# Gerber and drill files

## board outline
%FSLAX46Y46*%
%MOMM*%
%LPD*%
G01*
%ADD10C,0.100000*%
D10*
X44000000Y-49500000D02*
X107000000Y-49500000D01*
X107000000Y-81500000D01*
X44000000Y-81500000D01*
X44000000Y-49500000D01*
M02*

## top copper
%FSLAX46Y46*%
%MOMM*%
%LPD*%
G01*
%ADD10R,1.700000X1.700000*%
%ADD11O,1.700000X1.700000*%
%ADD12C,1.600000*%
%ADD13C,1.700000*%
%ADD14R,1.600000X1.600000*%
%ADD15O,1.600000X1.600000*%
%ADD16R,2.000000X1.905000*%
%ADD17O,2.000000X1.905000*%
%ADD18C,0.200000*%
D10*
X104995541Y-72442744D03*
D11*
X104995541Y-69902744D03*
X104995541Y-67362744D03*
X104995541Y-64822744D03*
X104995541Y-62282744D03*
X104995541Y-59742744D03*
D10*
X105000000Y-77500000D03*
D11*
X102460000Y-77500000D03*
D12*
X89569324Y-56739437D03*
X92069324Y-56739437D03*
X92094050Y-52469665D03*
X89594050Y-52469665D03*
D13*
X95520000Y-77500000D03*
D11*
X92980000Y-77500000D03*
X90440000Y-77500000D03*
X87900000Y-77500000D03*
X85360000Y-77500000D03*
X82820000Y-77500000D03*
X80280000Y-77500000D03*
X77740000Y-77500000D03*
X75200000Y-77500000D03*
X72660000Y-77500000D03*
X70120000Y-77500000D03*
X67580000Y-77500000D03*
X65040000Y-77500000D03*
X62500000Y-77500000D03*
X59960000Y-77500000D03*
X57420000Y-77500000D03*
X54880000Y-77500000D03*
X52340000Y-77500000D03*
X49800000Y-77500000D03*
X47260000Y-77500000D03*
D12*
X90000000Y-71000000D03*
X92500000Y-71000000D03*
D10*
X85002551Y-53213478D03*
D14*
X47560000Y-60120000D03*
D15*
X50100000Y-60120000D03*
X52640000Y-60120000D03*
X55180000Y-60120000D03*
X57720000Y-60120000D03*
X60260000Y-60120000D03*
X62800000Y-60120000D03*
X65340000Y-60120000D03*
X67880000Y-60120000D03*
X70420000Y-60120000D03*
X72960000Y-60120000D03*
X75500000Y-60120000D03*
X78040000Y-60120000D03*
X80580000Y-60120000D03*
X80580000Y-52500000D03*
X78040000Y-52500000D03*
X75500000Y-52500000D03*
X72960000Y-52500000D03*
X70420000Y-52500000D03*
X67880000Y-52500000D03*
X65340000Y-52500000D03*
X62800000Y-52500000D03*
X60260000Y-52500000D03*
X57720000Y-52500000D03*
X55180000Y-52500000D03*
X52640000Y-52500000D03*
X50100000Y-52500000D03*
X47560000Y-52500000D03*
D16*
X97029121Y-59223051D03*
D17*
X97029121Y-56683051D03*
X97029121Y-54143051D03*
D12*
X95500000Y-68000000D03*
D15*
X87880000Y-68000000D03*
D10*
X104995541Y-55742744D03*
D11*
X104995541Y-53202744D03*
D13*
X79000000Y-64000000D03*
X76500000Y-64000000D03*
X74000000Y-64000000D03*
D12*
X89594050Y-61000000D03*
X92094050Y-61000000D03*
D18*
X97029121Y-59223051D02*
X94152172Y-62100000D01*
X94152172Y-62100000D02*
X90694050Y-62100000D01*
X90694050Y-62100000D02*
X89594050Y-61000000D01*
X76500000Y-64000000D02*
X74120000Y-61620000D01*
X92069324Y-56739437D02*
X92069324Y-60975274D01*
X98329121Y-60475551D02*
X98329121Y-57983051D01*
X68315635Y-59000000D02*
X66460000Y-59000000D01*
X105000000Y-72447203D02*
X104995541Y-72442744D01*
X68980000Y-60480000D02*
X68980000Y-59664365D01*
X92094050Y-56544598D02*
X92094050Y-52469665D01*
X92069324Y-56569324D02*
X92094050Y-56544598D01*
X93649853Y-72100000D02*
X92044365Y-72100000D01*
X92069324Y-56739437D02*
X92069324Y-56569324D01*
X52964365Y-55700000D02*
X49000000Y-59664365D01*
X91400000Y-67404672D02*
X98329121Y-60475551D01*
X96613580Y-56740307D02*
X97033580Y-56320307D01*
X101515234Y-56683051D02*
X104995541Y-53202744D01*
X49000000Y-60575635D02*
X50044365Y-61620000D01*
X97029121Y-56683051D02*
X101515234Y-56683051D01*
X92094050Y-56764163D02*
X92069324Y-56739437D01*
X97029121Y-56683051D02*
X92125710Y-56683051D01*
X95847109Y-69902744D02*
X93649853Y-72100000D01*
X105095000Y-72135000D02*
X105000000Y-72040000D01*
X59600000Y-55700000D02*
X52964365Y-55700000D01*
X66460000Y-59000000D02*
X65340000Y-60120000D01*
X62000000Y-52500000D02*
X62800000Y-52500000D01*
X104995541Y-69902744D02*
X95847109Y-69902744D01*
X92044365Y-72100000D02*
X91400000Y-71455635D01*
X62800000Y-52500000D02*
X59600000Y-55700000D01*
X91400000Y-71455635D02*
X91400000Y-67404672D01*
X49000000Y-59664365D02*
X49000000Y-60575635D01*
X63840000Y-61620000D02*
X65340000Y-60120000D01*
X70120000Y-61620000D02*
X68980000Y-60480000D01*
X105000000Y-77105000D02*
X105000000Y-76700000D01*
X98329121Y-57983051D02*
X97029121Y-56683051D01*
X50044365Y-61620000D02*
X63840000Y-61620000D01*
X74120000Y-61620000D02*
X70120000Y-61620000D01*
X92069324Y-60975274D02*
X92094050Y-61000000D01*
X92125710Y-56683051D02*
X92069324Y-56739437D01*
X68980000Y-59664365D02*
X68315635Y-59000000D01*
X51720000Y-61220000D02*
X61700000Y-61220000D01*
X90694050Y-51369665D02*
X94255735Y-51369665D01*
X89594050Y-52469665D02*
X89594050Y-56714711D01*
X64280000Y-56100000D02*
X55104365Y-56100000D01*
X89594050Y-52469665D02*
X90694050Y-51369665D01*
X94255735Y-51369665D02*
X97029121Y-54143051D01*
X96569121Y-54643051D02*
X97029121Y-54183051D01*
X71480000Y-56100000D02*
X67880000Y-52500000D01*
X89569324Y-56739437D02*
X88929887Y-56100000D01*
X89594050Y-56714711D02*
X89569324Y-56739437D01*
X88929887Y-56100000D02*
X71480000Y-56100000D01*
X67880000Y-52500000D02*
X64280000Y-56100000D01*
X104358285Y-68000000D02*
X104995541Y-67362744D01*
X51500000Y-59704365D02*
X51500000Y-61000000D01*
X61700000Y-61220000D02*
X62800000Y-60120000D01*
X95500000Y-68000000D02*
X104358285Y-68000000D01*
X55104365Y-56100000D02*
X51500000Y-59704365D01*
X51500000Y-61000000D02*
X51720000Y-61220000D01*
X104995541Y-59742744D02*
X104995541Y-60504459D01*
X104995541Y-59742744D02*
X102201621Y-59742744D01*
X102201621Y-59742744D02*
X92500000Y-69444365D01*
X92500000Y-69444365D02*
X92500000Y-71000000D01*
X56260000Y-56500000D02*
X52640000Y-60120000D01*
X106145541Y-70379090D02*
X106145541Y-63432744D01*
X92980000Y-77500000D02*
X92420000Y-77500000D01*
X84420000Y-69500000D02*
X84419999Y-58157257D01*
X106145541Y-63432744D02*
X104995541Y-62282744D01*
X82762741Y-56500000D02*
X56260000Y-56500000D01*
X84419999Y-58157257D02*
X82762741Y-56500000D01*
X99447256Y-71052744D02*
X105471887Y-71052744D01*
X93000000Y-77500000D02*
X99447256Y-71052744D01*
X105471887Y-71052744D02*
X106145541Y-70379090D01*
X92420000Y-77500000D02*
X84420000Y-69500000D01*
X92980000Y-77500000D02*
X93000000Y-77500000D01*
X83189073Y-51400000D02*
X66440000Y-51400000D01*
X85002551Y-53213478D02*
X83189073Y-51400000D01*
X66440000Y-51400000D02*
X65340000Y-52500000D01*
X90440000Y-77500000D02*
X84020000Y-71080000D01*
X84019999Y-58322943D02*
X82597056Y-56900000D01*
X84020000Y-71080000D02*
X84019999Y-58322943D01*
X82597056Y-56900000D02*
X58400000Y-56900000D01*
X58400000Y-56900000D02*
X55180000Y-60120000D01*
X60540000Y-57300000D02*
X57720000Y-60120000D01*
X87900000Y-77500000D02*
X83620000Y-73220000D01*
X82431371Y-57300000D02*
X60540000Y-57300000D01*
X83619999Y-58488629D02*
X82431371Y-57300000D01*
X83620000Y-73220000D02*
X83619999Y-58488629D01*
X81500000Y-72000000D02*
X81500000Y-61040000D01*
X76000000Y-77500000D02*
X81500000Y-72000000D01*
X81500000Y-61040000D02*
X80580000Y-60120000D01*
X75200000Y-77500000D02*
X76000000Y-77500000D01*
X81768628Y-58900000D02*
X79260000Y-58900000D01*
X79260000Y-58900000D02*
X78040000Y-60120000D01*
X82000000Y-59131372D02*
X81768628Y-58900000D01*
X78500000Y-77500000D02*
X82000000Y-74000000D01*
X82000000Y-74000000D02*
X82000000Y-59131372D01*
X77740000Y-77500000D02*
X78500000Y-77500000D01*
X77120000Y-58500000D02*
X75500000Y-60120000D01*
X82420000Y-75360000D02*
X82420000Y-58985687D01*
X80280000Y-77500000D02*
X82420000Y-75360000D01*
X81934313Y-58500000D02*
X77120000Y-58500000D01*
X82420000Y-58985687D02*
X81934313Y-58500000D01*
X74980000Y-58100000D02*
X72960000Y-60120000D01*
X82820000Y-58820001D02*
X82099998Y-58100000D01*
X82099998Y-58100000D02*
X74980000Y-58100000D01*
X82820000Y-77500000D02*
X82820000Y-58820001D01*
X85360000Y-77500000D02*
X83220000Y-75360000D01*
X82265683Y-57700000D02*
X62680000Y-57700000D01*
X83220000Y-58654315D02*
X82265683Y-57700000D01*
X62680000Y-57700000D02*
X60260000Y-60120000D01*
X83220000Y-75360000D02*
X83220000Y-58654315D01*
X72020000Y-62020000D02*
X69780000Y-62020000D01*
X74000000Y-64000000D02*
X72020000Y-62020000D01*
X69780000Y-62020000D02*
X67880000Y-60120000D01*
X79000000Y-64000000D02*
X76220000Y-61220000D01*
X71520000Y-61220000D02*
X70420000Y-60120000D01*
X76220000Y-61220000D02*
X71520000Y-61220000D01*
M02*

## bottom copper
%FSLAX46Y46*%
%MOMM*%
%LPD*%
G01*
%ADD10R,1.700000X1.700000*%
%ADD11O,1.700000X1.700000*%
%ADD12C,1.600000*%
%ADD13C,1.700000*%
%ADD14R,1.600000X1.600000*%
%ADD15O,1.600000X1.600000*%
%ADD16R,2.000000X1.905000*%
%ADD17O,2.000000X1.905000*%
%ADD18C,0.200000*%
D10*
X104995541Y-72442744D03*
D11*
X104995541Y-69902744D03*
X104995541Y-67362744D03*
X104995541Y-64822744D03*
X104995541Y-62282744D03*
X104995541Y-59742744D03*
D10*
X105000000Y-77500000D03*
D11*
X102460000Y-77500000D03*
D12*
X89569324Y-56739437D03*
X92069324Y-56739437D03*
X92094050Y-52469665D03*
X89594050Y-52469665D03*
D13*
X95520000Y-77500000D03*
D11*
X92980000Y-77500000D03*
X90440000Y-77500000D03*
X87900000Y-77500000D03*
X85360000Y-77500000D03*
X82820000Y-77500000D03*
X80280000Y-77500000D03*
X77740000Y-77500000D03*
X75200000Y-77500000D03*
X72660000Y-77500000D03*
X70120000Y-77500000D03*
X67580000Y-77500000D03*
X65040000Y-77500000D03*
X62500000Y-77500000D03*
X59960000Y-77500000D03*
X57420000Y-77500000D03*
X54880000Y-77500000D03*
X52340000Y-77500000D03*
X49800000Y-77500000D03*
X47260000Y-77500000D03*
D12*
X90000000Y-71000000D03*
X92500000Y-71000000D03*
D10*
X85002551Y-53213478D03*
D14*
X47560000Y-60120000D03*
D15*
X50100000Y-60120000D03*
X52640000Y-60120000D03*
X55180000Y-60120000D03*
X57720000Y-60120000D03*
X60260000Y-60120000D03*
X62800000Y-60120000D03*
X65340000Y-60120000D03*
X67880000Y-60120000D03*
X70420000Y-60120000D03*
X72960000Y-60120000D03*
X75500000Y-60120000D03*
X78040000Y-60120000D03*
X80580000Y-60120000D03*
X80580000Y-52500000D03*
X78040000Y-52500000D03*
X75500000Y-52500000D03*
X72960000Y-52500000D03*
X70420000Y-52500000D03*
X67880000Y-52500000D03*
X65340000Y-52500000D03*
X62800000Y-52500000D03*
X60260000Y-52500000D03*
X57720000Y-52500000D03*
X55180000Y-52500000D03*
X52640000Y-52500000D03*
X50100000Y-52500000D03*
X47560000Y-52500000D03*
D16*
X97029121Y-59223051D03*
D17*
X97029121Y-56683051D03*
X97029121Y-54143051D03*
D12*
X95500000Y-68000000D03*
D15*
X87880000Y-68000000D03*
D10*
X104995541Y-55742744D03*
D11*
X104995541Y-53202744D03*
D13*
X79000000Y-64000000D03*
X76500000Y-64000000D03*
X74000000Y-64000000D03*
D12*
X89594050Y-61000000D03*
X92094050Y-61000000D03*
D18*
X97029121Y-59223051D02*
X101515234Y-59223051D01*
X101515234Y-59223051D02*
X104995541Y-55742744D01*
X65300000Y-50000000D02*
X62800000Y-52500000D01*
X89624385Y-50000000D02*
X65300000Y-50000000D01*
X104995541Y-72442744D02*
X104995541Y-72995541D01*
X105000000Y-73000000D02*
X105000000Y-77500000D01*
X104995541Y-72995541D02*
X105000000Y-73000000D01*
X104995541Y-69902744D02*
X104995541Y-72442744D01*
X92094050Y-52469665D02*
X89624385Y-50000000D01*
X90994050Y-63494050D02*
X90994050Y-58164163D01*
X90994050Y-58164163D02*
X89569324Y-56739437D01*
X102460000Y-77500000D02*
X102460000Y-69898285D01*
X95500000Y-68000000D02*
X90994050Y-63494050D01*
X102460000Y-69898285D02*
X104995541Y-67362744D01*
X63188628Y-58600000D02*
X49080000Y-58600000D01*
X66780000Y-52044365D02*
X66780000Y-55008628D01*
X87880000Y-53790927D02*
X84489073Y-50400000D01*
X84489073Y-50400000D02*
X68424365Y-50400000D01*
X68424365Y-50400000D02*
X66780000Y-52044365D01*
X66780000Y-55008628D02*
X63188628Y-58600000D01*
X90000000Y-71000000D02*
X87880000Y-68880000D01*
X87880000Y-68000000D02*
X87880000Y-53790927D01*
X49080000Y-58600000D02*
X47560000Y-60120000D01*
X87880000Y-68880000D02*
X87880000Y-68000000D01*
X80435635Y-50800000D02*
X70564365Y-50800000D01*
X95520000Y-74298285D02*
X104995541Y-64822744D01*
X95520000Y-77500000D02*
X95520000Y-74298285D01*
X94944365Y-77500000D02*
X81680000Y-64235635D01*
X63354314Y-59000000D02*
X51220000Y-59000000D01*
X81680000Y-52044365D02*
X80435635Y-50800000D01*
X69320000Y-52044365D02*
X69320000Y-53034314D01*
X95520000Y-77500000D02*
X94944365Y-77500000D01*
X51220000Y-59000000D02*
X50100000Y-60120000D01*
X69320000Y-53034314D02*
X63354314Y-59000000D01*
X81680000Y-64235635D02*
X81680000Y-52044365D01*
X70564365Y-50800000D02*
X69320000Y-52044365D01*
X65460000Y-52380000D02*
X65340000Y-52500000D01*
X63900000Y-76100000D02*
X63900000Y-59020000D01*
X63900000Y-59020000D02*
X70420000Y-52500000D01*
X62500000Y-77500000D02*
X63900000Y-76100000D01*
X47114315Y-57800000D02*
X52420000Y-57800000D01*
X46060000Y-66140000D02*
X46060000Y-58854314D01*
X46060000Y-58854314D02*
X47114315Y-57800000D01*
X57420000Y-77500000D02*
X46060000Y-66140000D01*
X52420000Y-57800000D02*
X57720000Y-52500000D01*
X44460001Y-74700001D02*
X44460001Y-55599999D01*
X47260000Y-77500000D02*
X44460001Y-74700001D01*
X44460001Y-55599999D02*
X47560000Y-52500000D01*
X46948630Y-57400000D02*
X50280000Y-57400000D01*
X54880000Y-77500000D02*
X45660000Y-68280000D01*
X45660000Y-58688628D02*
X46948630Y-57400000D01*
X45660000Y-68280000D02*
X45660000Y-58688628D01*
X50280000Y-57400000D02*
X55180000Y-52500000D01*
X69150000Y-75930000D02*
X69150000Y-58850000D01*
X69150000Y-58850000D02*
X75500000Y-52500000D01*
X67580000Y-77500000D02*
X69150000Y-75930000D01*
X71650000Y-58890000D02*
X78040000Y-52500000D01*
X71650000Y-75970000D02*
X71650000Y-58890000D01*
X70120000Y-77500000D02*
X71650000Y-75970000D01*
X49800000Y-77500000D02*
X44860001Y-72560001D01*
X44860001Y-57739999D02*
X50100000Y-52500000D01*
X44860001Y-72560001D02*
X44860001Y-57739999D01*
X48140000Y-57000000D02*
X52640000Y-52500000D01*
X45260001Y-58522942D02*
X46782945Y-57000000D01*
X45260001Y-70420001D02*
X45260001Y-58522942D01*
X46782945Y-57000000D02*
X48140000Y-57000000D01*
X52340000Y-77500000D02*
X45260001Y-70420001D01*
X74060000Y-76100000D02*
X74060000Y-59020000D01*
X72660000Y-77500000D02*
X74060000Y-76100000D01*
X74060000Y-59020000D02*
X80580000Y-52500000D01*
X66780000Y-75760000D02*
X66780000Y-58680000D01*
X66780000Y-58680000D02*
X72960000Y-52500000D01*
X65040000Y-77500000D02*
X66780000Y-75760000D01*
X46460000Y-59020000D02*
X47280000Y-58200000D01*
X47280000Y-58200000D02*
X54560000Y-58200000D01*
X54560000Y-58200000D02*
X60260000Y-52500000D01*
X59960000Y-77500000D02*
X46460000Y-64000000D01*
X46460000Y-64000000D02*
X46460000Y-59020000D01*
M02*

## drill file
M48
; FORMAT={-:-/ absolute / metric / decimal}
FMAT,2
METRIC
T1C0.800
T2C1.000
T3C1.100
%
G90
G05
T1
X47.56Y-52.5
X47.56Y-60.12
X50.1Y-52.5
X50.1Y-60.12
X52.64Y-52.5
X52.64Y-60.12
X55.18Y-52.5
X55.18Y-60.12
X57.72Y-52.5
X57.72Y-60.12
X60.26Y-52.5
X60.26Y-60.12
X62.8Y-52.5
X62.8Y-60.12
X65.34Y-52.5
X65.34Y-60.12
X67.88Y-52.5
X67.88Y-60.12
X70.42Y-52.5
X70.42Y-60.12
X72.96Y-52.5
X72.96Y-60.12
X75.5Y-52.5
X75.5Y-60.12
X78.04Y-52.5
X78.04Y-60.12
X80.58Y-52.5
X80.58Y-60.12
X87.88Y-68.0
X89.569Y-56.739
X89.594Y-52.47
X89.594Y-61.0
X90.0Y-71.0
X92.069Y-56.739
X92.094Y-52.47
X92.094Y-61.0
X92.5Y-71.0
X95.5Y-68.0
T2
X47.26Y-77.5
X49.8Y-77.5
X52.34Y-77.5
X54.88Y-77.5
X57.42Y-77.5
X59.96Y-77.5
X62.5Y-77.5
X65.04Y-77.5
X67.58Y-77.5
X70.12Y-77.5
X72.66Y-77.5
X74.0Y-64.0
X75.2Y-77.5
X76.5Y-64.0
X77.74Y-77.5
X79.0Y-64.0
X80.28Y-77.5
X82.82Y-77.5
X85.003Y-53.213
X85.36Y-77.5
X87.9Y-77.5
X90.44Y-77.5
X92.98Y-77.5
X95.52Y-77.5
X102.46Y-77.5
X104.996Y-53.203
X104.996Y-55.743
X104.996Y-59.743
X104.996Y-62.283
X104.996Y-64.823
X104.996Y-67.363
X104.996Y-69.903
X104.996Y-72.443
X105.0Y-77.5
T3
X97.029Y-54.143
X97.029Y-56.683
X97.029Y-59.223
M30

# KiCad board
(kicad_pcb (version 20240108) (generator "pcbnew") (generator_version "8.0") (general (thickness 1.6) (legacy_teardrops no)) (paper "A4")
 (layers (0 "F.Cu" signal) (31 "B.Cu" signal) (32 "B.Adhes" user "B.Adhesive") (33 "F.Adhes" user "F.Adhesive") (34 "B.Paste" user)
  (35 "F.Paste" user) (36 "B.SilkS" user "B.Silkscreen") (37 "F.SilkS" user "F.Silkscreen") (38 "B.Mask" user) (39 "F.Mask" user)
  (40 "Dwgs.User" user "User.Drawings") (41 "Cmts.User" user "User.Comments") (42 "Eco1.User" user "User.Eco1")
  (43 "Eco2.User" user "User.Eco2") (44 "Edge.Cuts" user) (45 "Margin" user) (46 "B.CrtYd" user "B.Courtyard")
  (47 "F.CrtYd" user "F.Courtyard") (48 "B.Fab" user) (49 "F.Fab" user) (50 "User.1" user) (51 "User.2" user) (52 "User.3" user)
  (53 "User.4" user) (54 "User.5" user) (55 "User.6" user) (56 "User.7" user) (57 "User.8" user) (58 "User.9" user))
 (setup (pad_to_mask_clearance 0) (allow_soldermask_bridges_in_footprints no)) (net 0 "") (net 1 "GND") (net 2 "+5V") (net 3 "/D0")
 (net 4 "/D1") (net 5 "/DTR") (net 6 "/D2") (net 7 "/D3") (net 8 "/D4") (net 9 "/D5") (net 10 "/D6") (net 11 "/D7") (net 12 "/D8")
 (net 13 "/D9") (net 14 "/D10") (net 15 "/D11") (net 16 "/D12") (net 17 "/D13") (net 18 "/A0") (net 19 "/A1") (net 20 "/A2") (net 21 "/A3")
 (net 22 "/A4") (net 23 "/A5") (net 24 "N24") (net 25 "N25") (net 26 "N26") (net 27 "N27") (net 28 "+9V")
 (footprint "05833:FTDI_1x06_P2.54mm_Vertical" (layer "F.Cu") (at 104.995541 72.442744 180)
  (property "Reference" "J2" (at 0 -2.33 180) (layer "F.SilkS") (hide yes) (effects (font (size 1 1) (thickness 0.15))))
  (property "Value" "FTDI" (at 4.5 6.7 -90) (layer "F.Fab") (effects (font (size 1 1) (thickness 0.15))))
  (pad "1" thru_hole rect (at 0 0 180) (size 1.7 1.7) (drill 1) (layers "*.Cu" "*.Mask") (remove_unused_layers no) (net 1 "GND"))
  (pad "2" thru_hole oval (at 0 2.54 180) (size 1.7 1.7) (drill 1) (layers "*.Cu" "*.Mask") (remove_unused_layers no) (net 1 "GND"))
  (pad "3" thru_hole oval (at 0 5.08 180) (size 1.7 1.7) (drill 1) (layers "*.Cu" "*.Mask") (remove_unused_layers no) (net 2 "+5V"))
  (pad "4" thru_hole oval (at 0 7.62 180) (size 1.7 1.7) (drill 1) (layers "*.Cu" "*.Mask") (remove_unused_layers no) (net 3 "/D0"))
  (pad "5" thru_hole oval (at 0 10.16 180) (size 1.7 1.7) (drill 1) (layers "*.Cu" "*.Mask") (remove_unused_layers no) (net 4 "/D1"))
  (pad "6" thru_hole oval (at 0 12.7 180) (size 1.7 1.7) (drill 1) (layers "*.Cu" "*.Mask") (remove_unused_layers no) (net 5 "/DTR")))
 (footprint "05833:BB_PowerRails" (layer "F.Cu") (at 105 77.5 -90)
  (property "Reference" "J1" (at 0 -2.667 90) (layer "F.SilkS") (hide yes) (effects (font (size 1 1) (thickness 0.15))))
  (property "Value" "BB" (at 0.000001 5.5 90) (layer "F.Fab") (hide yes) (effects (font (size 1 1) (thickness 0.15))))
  (pad "1" thru_hole rect (at 0 0 270) (size 1.7 1.7) (drill 1) (layers "*.Cu" "*.Mask") (remove_unused_layers no) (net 1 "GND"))
  (pad "2" thru_hole oval (at 0 2.54 270) (size 1.7 1.7) (drill 1) (layers "*.Cu" "*.Mask") (remove_unused_layers no) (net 2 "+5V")))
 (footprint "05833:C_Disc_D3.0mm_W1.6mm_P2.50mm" (layer "F.Cu") (at 89.569324 56.739437)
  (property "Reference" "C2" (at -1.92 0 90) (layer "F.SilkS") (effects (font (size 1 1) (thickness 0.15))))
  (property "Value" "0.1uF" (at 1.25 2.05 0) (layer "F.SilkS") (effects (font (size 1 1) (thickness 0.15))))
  (pad "1" thru_hole circle (at 0 0) (size 1.6 1.6) (drill 0.8) (layers "*.Cu" "*.Mask") (remove_unused_layers no) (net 2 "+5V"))
  (pad "2" thru_hole circle (at 2.5 0) (size 1.6 1.6) (drill 0.8) (layers "*.Cu" "*.Mask") (remove_unused_layers no) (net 1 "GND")))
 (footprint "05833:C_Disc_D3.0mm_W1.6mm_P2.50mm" (layer "F.Cu") (at 92.09405 52.469665 180)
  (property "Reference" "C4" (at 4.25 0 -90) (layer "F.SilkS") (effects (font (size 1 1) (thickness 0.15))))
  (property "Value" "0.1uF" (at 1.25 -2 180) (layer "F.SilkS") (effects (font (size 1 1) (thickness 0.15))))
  (pad "1" thru_hole circle (at 0 0 180) (size 1.6 1.6) (drill 0.8) (layers "*.Cu" "*.Mask") (remove_unused_layers no) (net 1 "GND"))
  (pad "2" thru_hole circle (at 2.5 0 180) (size 1.6 1.6) (drill 0.8) (layers "*.Cu" "*.Mask") (remove_unused_layers no) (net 2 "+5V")))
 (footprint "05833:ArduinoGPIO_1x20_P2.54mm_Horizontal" (layer "F.Cu") (at 95.52 77.5 -90)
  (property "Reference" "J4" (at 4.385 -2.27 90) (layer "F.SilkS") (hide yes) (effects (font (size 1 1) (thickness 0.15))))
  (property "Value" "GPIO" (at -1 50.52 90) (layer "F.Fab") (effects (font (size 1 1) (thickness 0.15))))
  (pad "1" thru_hole circle (at 0 0 270) (size 1.7 1.7) (drill 1) (layers "*.Cu" "*.Mask") (remove_unused_layers no) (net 3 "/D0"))
  (pad "2" thru_hole oval (at 0 2.54 270) (size 1.7 1.7) (drill 1) (layers "*.Cu" "*.Mask") (remove_unused_layers no) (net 4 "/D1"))
  (pad "3" thru_hole oval (at 0 5.08 270) (size 1.7 1.7) (drill 1) (layers "*.Cu" "*.Mask") (remove_unused_layers no) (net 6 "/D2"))
  (pad "4" thru_hole oval (at 0 7.62 270) (size 1.7 1.7) (drill 1) (layers "*.Cu" "*.Mask") (remove_unused_layers no) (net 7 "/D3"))
  (pad "5" thru_hole oval (at 0 10.16 270) (size 1.7 1.7) (drill 1) (layers "*.Cu" "*.Mask") (remove_unused_layers no) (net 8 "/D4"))
  (pad "6" thru_hole oval (at 0 12.7 270) (size 1.7 1.7) (drill 1) (layers "*.Cu" "*.Mask") (remove_unused_layers no) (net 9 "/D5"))
  (pad "7" thru_hole oval (at 0 15.24 270) (size 1.7 1.7) (drill 1) (layers "*.Cu" "*.Mask") (remove_unused_layers no) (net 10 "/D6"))
  (pad "8" thru_hole oval (at 0 17.78 270) (size 1.7 1.7) (drill 1) (layers "*.Cu" "*.Mask") (remove_unused_layers no) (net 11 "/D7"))
  (pad "9" thru_hole oval (at 0 20.32 270) (size 1.7 1.7) (drill 1) (layers "*.Cu" "*.Mask") (remove_unused_layers no) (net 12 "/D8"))
  (pad "10" thru_hole oval (at 0 22.86 270) (size 1.7 1.7) (drill 1) (layers "*.Cu" "*.Mask") (remove_unused_layers no) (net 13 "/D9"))
  (pad "11" thru_hole oval (at 0 25.4 270) (size 1.7 1.7) (drill 1) (layers "*.Cu" "*.Mask") (remove_unused_layers no) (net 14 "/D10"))
  (pad "12" thru_hole oval (at 0 27.94 270) (size 1.7 1.7) (drill 1) (layers "*.Cu" "*.Mask") (remove_unused_layers no) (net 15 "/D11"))
  (pad "13" thru_hole oval (at 0 30.48 270) (size 1.7 1.7) (drill 1) (layers "*.Cu" "*.Mask") (remove_unused_layers no) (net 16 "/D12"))
  (pad "14" thru_hole oval (at 0 33.02 270) (size 1.7 1.7) (drill 1) (layers "*.Cu" "*.Mask") (remove_unused_layers no) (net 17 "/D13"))
  (pad "15" thru_hole oval (at 0 35.56 270) (size 1.7 1.7) (drill 1) (layers "*.Cu" "*.Mask") (remove_unused_layers no) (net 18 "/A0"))
  (pad "16" thru_hole oval (at 0 38.1 270) (size 1.7 1.7) (drill 1) (layers "*.Cu" "*.Mask") (remove_unused_layers no) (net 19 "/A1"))
  (pad "17" thru_hole oval (at 0 40.64 270) (size 1.7 1.7) (drill 1) (layers "*.Cu" "*.Mask") (remove_unused_layers no) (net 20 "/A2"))
  (pad "18" thru_hole oval (at 0 43.18 270) (size 1.7 1.7) (drill 1) (layers "*.Cu" "*.Mask") (remove_unused_layers no) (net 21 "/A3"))
  (pad "19" thru_hole oval (at 0 45.72 270) (size 1.7 1.7) (drill 1) (layers "*.Cu" "*.Mask") (remove_unused_layers no) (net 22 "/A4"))
  (pad "20" thru_hole oval (at 0 48.26 270) (size 1.7 1.7) (drill 1) (layers "*.Cu" "*.Mask") (remove_unused_layers no) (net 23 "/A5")))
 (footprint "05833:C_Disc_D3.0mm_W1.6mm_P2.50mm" (layer "F.Cu") (at 90 71)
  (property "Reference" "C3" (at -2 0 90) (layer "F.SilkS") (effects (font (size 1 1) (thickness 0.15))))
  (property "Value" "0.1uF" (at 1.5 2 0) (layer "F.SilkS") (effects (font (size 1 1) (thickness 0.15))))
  (pad "1" thru_hole circle (at 0 0) (size 1.6 1.6) (drill 0.8) (layers "*.Cu" "*.Mask") (remove_unused_layers no) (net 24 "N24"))
  (pad "2" thru_hole circle (at 2.5 0) (size 1.6 1.6) (drill 0.8) (layers "*.Cu" "*.Mask") (remove_unused_layers no) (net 5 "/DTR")))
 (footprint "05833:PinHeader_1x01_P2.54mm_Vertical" (layer "F.Cu") (at 85.002551 53.213478)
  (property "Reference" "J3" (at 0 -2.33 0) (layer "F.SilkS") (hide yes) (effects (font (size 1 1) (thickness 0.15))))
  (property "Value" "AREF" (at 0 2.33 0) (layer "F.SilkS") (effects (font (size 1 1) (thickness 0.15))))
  (pad "1" thru_hole rect (at 0 0) (size 1.7 1.7) (drill 1) (layers "*.Cu" "*.Mask") (remove_unused_layers no) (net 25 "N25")))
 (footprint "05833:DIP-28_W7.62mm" (layer "F.Cu") (at 47.56 60.12 90)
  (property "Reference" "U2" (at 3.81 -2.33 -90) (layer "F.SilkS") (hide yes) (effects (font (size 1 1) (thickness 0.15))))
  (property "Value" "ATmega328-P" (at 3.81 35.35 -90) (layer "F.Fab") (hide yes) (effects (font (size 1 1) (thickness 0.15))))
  (pad "1" thru_hole rect (at 0 0 90) (size 1.6 1.6) (drill 0.8) (layers "*.Cu" "*.Mask") (remove_unused_layers no) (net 24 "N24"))
  (pad "2" thru_hole oval (at 0 2.54 90) (size 1.6 1.6) (drill 0.8) (layers "*.Cu" "*.Mask") (remove_unused_layers no) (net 3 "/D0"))
  (pad "3" thru_hole oval (at 0 5.08 90) (size 1.6 1.6) (drill 0.8) (layers "*.Cu" "*.Mask") (remove_unused_layers no) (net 4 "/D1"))
  (pad "4" thru_hole oval (at 0 7.62 90) (size 1.6 1.6) (drill 0.8) (layers "*.Cu" "*.Mask") (remove_unused_layers no) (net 6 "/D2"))
  (pad "5" thru_hole oval (at 0 10.16 90) (size 1.6 1.6) (drill 0.8) (layers "*.Cu" "*.Mask") (remove_unused_layers no) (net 7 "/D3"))
  (pad "6" thru_hole oval (at 0 12.7 90) (size 1.6 1.6) (drill 0.8) (layers "*.Cu" "*.Mask") (remove_unused_layers no) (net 8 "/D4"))
  (pad "7" thru_hole oval (at 0 15.24 90) (size 1.6 1.6) (drill 0.8) (layers "*.Cu" "*.Mask") (remove_unused_layers no) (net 2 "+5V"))
  (pad "8" thru_hole oval (at 0 17.78 90) (size 1.6 1.6) (drill 0.8) (layers "*.Cu" "*.Mask") (remove_unused_layers no) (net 1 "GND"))
  (pad "9" thru_hole oval (at 0 20.32 90) (size 1.6 1.6) (drill 0.8) (layers "*.Cu" "*.Mask") (remove_unused_layers no) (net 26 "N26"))
  (pad "10" thru_hole oval (at 0 22.86 90) (size 1.6 1.6) (drill 0.8) (layers "*.Cu" "*.Mask") (remove_unused_layers no) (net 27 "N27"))
  (pad "11" thru_hole oval (at 0 25.4 90) (size 1.6 1.6) (drill 0.8) (layers "*.Cu" "*.Mask") (remove_unused_layers no) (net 9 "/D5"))
  (pad "12" thru_hole oval (at 0 27.94 90) (size 1.6 1.6) (drill 0.8) (layers "*.Cu" "*.Mask") (remove_unused_layers no) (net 10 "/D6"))
  (pad "13" thru_hole oval (at 0 30.48 90) (size 1.6 1.6) (drill 0.8) (layers "*.Cu" "*.Mask") (remove_unused_layers no) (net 11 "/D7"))
  (pad "14" thru_hole oval (at 0 33.02 90) (size 1.6 1.6) (drill 0.8) (layers "*.Cu" "*.Mask") (remove_unused_layers no) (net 12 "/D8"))
  (pad "15" thru_hole oval (at 7.62 33.02 90) (size 1.6 1.6) (drill 0.8) (layers "*.Cu" "*.Mask") (remove_unused_layers no) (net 13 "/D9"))
  (pad "16" thru_hole oval (at 7.62 30.48 90) (size 1.6 1.6) (drill 0.8) (layers "*.Cu" "*.Mask") (remove_unused_layers no) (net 14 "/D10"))
  (pad "17" thru_hole oval (at 7.62 27.94 90) (size 1.6 1.6) (drill 0.8) (layers "*.Cu" "*.Mask") (remove_unused_layers no) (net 15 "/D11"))
  (pad "18" thru_hole oval (at 7.62 25.4 90) (size 1.6 1.6) (drill 0.8) (layers "*.Cu" "*.Mask") (remove_unused_layers no) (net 16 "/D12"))
  (pad "19" thru_hole oval (at 7.62 22.86 90) (size 1.6 1.6) (drill 0.8) (layers "*.Cu" "*.Mask") (remove_unused_layers no) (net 17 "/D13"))
  (pad "20" thru_hole oval (at 7.62 20.32 90) (size 1.6 1.6) (drill 0.8) (layers "*.Cu" "*.Mask") (remove_unused_layers no) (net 2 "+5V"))
  (pad "21" thru_hole oval (at 7.62 17.78 90) (size 1.6 1.6) (drill 0.8) (layers "*.Cu" "*.Mask") (remove_unused_layers no) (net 25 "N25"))
  (pad "22" thru_hole oval (at 7.62 15.24 90) (size 1.6 1.6) (drill 0.8) (layers "*.Cu" "*.Mask") (remove_unused_layers no) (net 1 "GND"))
  (pad "23" thru_hole oval (at 7.62 12.7 90) (size 1.6 1.6) (drill 0.8) (layers "*.Cu" "*.Mask") (remove_unused_layers no) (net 18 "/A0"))
  (pad "24" thru_hole oval (at 7.62 10.16 90) (size 1.6 1.6) (drill 0.8) (layers "*.Cu" "*.Mask") (remove_unused_layers no) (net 19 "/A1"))
  (pad "25" thru_hole oval (at 7.62 7.62 90) (size 1.6 1.6) (drill 0.8) (layers "*.Cu" "*.Mask") (remove_unused_layers no) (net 20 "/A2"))
  (pad "26" thru_hole oval (at 7.62 5.08 90) (size 1.6 1.6) (drill 0.8) (layers "*.Cu" "*.Mask") (remove_unused_layers no) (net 21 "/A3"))
  (pad "27" thru_hole oval (at 7.62 2.54 90) (size 1.6 1.6) (drill 0.8) (layers "*.Cu" "*.Mask") (remove_unused_layers no) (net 22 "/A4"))
  (pad "28" thru_hole oval (at 7.62 0 90) (size 1.6 1.6) (drill 0.8) (layers "*.Cu" "*.Mask") (remove_unused_layers no) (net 23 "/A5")))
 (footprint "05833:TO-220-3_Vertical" (layer "F.Cu") (at 97.029121 59.223051 90)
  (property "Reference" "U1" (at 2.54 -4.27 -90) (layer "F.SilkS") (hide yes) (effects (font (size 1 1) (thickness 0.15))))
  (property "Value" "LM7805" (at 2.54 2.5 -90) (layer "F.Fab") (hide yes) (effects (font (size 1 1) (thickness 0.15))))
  (pad "1" thru_hole rect (at 0 0 90) (size 1.905 2) (drill 1.1) (layers "*.Cu" "*.Mask") (remove_unused_layers no) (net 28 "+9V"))
  (pad "2" thru_hole oval (at 2.54 0 90) (size 1.905 2) (drill 1.1) (layers "*.Cu" "*.Mask") (remove_unused_layers no) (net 1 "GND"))
  (pad "3" thru_hole oval (at 5.08 0 90) (size 1.905 2) (drill 1.1) (layers "*.Cu" "*.Mask") (remove_unused_layers no) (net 2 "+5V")))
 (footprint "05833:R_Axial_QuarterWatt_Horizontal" (layer "F.Cu") (at 95.5 68 180)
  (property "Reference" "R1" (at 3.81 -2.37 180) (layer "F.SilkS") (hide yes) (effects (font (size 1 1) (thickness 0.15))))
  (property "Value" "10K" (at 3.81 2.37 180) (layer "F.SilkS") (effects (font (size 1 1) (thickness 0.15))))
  (pad "1" thru_hole circle (at 0 0 180) (size 1.6 1.6) (drill 0.8) (layers "*.Cu" "*.Mask") (remove_unused_layers no) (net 2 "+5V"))
  (pad "2" thru_hole oval (at 7.62 0 180) (size 1.6 1.6) (drill 0.8) (layers "*.Cu" "*.Mask") (remove_unused_layers no) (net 24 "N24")))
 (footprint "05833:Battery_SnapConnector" (layer "F.Cu") (at 104.995541 55.742744 180)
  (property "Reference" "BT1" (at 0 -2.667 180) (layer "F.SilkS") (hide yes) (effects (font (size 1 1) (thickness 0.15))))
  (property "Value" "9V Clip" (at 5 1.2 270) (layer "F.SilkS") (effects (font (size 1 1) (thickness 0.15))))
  (pad "1" thru_hole rect (at 0 0 180) (size 1.7 1.7) (drill 1) (layers "*.Cu" "*.Mask") (remove_unused_layers no) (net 28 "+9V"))
  (pad "2" thru_hole oval (at 0 2.54 180) (size 1.7 1.7) (drill 1) (layers "*.Cu" "*.Mask") (remove_unused_layers no) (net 1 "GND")))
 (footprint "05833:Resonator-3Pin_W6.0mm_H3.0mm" (layer "F.Cu") (at 79 64 180)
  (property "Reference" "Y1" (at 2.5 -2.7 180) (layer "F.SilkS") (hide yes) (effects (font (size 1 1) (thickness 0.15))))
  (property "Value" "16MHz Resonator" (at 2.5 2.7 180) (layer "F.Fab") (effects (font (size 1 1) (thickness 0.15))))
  (pad "1" thru_hole circle (at 0 0 180) (size 1.7 1.7) (drill 1) (layers "*.Cu" "*.Mask") (remove_unused_layers no) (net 27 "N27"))
  (pad "2" thru_hole circle (at 2.5 0 180) (size 1.7 1.7) (drill 1) (layers "*.Cu" "*.Mask") (remove_unused_layers no) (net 1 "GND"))
  (pad "3" thru_hole circle (at 5 0 180) (size 1.7 1.7) (drill 1) (layers "*.Cu" "*.Mask") (remove_unused_layers no) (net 26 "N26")))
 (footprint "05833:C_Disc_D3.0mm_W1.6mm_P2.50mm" (layer "F.Cu") (at 89.59405 61)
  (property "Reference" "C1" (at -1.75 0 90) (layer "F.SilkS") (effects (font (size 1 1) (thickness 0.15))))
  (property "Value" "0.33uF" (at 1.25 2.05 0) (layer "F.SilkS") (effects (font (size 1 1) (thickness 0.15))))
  (pad "1" thru_hole circle (at 0 0) (size 1.6 1.6) (drill 0.8) (layers "*.Cu" "*.Mask") (remove_unused_layers no) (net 28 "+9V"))
  (pad "2" thru_hole circle (at 2.5 0) (size 1.6 1.6) (drill 0.8) (layers "*.Cu" "*.Mask") (remove_unused_layers no) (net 1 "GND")))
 (gr_rect (start 44 49.5) (end 107 81.5) (stroke (width 0.1) (type default)) (fill none) (layer "Edge.Cuts"))
 (segment (start 97.029121 59.223051) (end 94.152172 62.1) (width 0.2) (layer "F.Cu") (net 28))
 (segment (start 94.152172 62.1) (end 90.69405 62.1) (width 0.2) (layer "F.Cu") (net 28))
 (segment (start 90.69405 62.1) (end 89.59405 61) (width 0.2) (layer "F.Cu") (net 28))
 (segment (start 97.029121 59.223051) (end 101.515234 59.223051) (width 0.2) (layer "B.Cu") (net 28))
 (segment (start 101.515234 59.223051) (end 104.995541 55.742744) (width 0.2) (layer "B.Cu") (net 28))
 (segment (start 76.5 64) (end 74.12 61.62) (width 0.2) (layer "F.Cu") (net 1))
 (segment (start 92.069324 56.739437) (end 92.069324 60.975274) (width 0.2) (layer "F.Cu") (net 1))
 (segment (start 98.329121 60.475551) (end 98.329121 57.983051) (width 0.2) (layer "F.Cu") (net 1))
 (segment (start 68.315635 59) (end 66.46 59) (width 0.2) (layer "F.Cu") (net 1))
 (segment (start 105 72.447203) (end 104.995541 72.442744) (width 0.2) (layer "F.Cu") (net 1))
 (segment (start 68.98 60.48) (end 68.98 59.664365) (width 0.2) (layer "F.Cu") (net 1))
 (segment (start 92.09405 56.544598) (end 92.09405 52.469665) (width 0.2) (layer "F.Cu") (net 1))
 (segment (start 92.069324 56.569324) (end 92.09405 56.544598) (width 0.2) (layer "F.Cu") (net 1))
 (segment (start 93.649853 72.1) (end 92.044365 72.1) (width 0.2) (layer "F.Cu") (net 1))
 (segment (start 92.069324 56.739437) (end 92.069324 56.569324) (width 0.2) (layer "F.Cu") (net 1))
 (segment (start 52.964365 55.7) (end 49 59.664365) (width 0.2) (layer "F.Cu") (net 1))
 (segment (start 91.4 67.404672) (end 98.329121 60.475551) (width 0.2) (layer "F.Cu") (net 1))
 (segment (start 96.61358 56.740307) (end 97.03358 56.320307) (width 0.2) (layer "F.Cu") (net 1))
 (segment (start 101.515234 56.683051) (end 104.995541 53.202744) (width 0.2) (layer "F.Cu") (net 1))
 (segment (start 49 60.575635) (end 50.044365 61.62) (width 0.2) (layer "F.Cu") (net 1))
 (segment (start 97.029121 56.683051) (end 101.515234 56.683051) (width 0.2) (layer "F.Cu") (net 1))
 (segment (start 92.09405 56.764163) (end 92.069324 56.739437) (width 0.2) (layer "F.Cu") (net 1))
 (segment (start 97.029121 56.683051) (end 92.12571 56.683051) (width 0.2) (layer "F.Cu") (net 1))
 (segment (start 95.847109 69.902744) (end 93.649853 72.1) (width 0.2) (layer "F.Cu") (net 1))
 (segment (start 105.095 72.135) (end 105 72.04) (width 0.2) (layer "F.Cu") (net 1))
 (segment (start 59.6 55.7) (end 52.964365 55.7) (width 0.2) (layer "F.Cu") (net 1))
 (segment (start 66.46 59) (end 65.34 60.12) (width 0.2) (layer "F.Cu") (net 1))
 (segment (start 62 52.5) (end 62.8 52.5) (width 0.2) (layer "F.Cu") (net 1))
 (segment (start 104.995541 69.902744) (end 95.847109 69.902744) (width 0.2) (layer "F.Cu") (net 1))
 (segment (start 92.044365 72.1) (end 91.4 71.455635) (width 0.2) (layer "F.Cu") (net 1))
 (segment (start 62.8 52.5) (end 59.6 55.7) (width 0.2) (layer "F.Cu") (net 1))
 (segment (start 91.4 71.455635) (end 91.4 67.404672) (width 0.2) (layer "F.Cu") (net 1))
 (segment (start 49 59.664365) (end 49 60.575635) (width 0.2) (layer "F.Cu") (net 1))
 (segment (start 63.84 61.62) (end 65.34 60.12) (width 0.2) (layer "F.Cu") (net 1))
 (segment (start 70.12 61.62) (end 68.98 60.48) (width 0.2) (layer "F.Cu") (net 1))
 (segment (start 105 77.105) (end 105 76.7) (width 0.2) (layer "F.Cu") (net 1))
 (segment (start 98.329121 57.983051) (end 97.029121 56.683051) (width 0.2) (layer "F.Cu") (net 1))
 (segment (start 50.044365 61.62) (end 63.84 61.62) (width 0.2) (layer "F.Cu") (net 1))
 (segment (start 74.12 61.62) (end 70.12 61.62) (width 0.2) (layer "F.Cu") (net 1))
 (segment (start 92.069324 60.975274) (end 92.09405 61) (width 0.2) (layer "F.Cu") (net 1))
 (segment (start 92.12571 56.683051) (end 92.069324 56.739437) (width 0.2) (layer "F.Cu") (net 1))
 (segment (start 68.98 59.664365) (end 68.315635 59) (width 0.2) (layer "F.Cu") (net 1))
 (segment (start 65.3 50) (end 62.8 52.5) (width 0.2) (layer "B.Cu") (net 1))
 (segment (start 89.624385 50) (end 65.3 50) (width 0.2) (layer "B.Cu") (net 1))
 (segment (start 104.995541 72.442744) (end 104.995541 72.995541) (width 0.2) (layer "B.Cu") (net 1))
 (segment (start 105 73) (end 105 77.5) (width 0.2) (layer "B.Cu") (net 1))
 (segment (start 104.995541 72.995541) (end 105 73) (width 0.2) (layer "B.Cu") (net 1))
 (segment (start 104.995541 69.902744) (end 104.995541 72.442744) (width 0.2) (layer "B.Cu") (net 1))
 (segment (start 92.09405 52.469665) (end 89.624385 50) (width 0.2) (layer "B.Cu") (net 1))
 (segment (start 51.72 61.22) (end 61.7 61.22) (width 0.2) (layer "F.Cu") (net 2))
 (segment (start 90.69405 51.369665) (end 94.255735 51.369665) (width 0.2) (layer "F.Cu") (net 2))
 (segment (start 89.59405 52.469665) (end 89.59405 56.714711) (width 0.2) (layer "F.Cu") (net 2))
 (segment (start 64.28 56.1) (end 55.104365 56.1) (width 0.2) (layer "F.Cu") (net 2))
 (segment (start 89.59405 52.469665) (end 90.69405 51.369665) (width 0.2) (layer "F.Cu") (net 2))
 (segment (start 94.255735 51.369665) (end 97.029121 54.143051) (width 0.2) (layer "F.Cu") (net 2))
 (segment (start 96.569121 54.643051) (end 97.029121 54.183051) (width 0.2) (layer "F.Cu") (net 2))
 (segment (start 71.48 56.1) (end 67.88 52.5) (width 0.2) (layer "F.Cu") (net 2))
 (segment (start 89.569324 56.739437) (end 88.929887 56.1) (width 0.2) (layer "F.Cu") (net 2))
 (segment (start 89.59405 56.714711) (end 89.569324 56.739437) (width 0.2) (layer "F.Cu") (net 2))
 (segment (start 88.929887 56.1) (end 71.48 56.1) (width 0.2) (layer "F.Cu") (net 2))
 (segment (start 67.88 52.5) (end 64.28 56.1) (width 0.2) (layer "F.Cu") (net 2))
 (segment (start 104.358285 68) (end 104.995541 67.362744) (width 0.2) (layer "F.Cu") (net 2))
 (segment (start 51.5 59.704365) (end 51.5 61) (width 0.2) (layer "F.Cu") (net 2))
 (segment (start 61.7 61.22) (end 62.8 60.12) (width 0.2) (layer "F.Cu") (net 2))
 (segment (start 95.5 68) (end 104.358285 68) (width 0.2) (layer "F.Cu") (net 2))
 (segment (start 55.104365 56.1) (end 51.5 59.704365) (width 0.2) (layer "F.Cu") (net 2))
 (segment (start 51.5 61) (end 51.72 61.22) (width 0.2) (layer "F.Cu") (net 2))
 (segment (start 90.99405 63.49405) (end 90.99405 58.164163) (width 0.2) (layer "B.Cu") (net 2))
 (segment (start 90.99405 58.164163) (end 89.569324 56.739437) (width 0.2) (layer "B.Cu") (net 2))
 (segment (start 102.46 77.5) (end 102.46 69.898285) (width 0.2) (layer "B.Cu") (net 2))
 (segment (start 95.5 68) (end 90.99405 63.49405) (width 0.2) (layer "B.Cu") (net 2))
 (segment (start 102.46 69.898285) (end 104.995541 67.362744) (width 0.2) (layer "B.Cu") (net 2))
 (segment (start 104.995541 59.742744) (end 104.995541 60.504459) (width 0.2) (layer "F.Cu") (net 5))
 (segment (start 104.995541 59.742744) (end 102.201621 59.742744) (width 0.2) (layer "F.Cu") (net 5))
 (segment (start 102.201621 59.742744) (end 92.5 69.444365) (width 0.2) (layer "F.Cu") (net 5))
 (segment (start 92.5 69.444365) (end 92.5 71) (width 0.2) (layer "F.Cu") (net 5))
 (segment (start 63.188628 58.6) (end 49.08 58.6) (width 0.2) (layer "B.Cu") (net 24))
 (segment (start 66.78 52.044365) (end 66.78 55.008628) (width 0.2) (layer "B.Cu") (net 24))
 (segment (start 87.88 53.790927) (end 84.489073 50.4) (width 0.2) (layer "B.Cu") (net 24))
 (segment (start 84.489073 50.4) (end 68.424365 50.4) (width 0.2) (layer "B.Cu") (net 24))
 (segment (start 68.424365 50.4) (end 66.78 52.044365) (width 0.2) (layer "B.Cu") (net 24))
 (segment (start 66.78 55.008628) (end 63.188628 58.6) (width 0.2) (layer "B.Cu") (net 24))
 (segment (start 90 71) (end 87.88 68.88) (width 0.2) (layer "B.Cu") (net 24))
 (segment (start 87.88 68) (end 87.88 53.790927) (width 0.2) (layer "B.Cu") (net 24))
 (segment (start 49.08 58.6) (end 47.56 60.12) (width 0.2) (layer "B.Cu") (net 24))
 (segment (start 87.88 68.88) (end 87.88 68) (width 0.2) (layer "B.Cu") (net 24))
 (segment (start 56.26 56.5) (end 52.64 60.12) (width 0.2) (layer "F.Cu") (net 4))
 (segment (start 106.145541 70.37909) (end 106.145541 63.432744) (width 0.2) (layer "F.Cu") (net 4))
 (segment (start 92.98 77.5) (end 92.42 77.5) (width 0.2) (layer "F.Cu") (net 4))
 (segment (start 84.42 69.5) (end 84.419999 58.157257) (width 0.2) (layer "F.Cu") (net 4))
 (segment (start 106.145541 63.432744) (end 104.995541 62.282744) (width 0.2) (layer "F.Cu") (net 4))
 (segment (start 82.762741 56.5) (end 56.26 56.5) (width 0.2) (layer "F.Cu") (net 4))
 (segment (start 84.419999 58.157257) (end 82.762741 56.5) (width 0.2) (layer "F.Cu") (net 4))
 (segment (start 99.447256 71.052744) (end 105.471887 71.052744) (width 0.2) (layer "F.Cu") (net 4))
 (segment (start 93 77.5) (end 99.447256 71.052744) (width 0.2) (layer "F.Cu") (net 4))
 (segment (start 105.471887 71.052744) (end 106.145541 70.37909) (width 0.2) (layer "F.Cu") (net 4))
 (segment (start 92.42 77.5) (end 84.42 69.5) (width 0.2) (layer "F.Cu") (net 4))
 (segment (start 92.98 77.5) (end 93 77.5) (width 0.2) (layer "F.Cu") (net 4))
 (segment (start 80.435635 50.8) (end 70.564365 50.8) (width 0.2) (layer "B.Cu") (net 3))
 (segment (start 95.52 74.298285) (end 104.995541 64.822744) (width 0.2) (layer "B.Cu") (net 3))
 (segment (start 95.52 77.5) (end 95.52 74.298285) (width 0.2) (layer "B.Cu") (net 3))
 (segment (start 94.944365 77.5) (end 81.68 64.235635) (width 0.2) (layer "B.Cu") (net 3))
 (segment (start 63.354314 59) (end 51.22 59) (width 0.2) (layer "B.Cu") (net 3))
 (segment (start 81.68 52.044365) (end 80.435635 50.8) (width 0.2) (layer "B.Cu") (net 3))
 (segment (start 69.32 52.044365) (end 69.32 53.034314) (width 0.2) (layer "B.Cu") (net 3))
 (segment (start 95.52 77.5) (end 94.944365 77.5) (width 0.2) (layer "B.Cu") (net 3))
 (segment (start 51.22 59) (end 50.1 60.12) (width 0.2) (layer "B.Cu") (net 3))
 (segment (start 69.32 53.034314) (end 63.354314 59) (width 0.2) (layer "B.Cu") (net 3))
 (segment (start 81.68 64.235635) (end 81.68 52.044365) (width 0.2) (layer "B.Cu") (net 3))
 (segment (start 70.564365 50.8) (end 69.32 52.044365) (width 0.2) (layer "B.Cu") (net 3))
 (segment (start 83.189073 51.4) (end 66.44 51.4) (width 0.2) (layer "F.Cu") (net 25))
 (segment (start 85.002551 53.213478) (end 83.189073 51.4) (width 0.2) (layer "F.Cu") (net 25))
 (segment (start 66.44 51.4) (end 65.34 52.5) (width 0.2) (layer "F.Cu") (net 25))
 (segment (start 65.46 52.38) (end 65.34 52.5) (width 0.2) (layer "B.Cu") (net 25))
 (segment (start 63.9 76.1) (end 63.9 59.02) (width 0.2) (layer "B.Cu") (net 17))
 (segment (start 63.9 59.02) (end 70.42 52.5) (width 0.2) (layer "B.Cu") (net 17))
 (segment (start 62.5 77.5) (end 63.9 76.1) (width 0.2) (layer "B.Cu") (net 17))
 (segment (start 47.114315 57.8) (end 52.42 57.8) (width 0.2) (layer "B.Cu") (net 19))
 (segment (start 46.06 66.14) (end 46.06 58.854314) (width 0.2) (layer "B.Cu") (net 19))
 (segment (start 46.06 58.854314) (end 47.114315 57.8) (width 0.2) (layer "B.Cu") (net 19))
 (segment (start 57.42 77.5) (end 46.06 66.14) (width 0.2) (layer "B.Cu") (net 19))
 (segment (start 52.42 57.8) (end 57.72 52.5) (width 0.2) (layer "B.Cu") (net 19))
 (segment (start 90.44 77.5) (end 84.02 71.08) (width 0.2) (layer "F.Cu") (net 6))
 (segment (start 84.019999 58.322943) (end 82.597056 56.9) (width 0.2) (layer "F.Cu") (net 6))
 (segment (start 84.02 71.08) (end 84.019999 58.322943) (width 0.2) (layer "F.Cu") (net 6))
 (segment (start 82.597056 56.9) (end 58.4 56.9) (width 0.2) (layer "F.Cu") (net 6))
 (segment (start 58.4 56.9) (end 55.18 60.12) (width 0.2) (layer "F.Cu") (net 6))
 (segment (start 44.460001 74.700001) (end 44.460001 55.599999) (width 0.2) (layer "B.Cu") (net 23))
 (segment (start 47.26 77.5) (end 44.460001 74.700001) (width 0.2) (layer "B.Cu") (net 23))
 (segment (start 44.460001 55.599999) (end 47.56 52.5) (width 0.2) (layer "B.Cu") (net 23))
 (segment (start 46.94863 57.4) (end 50.28 57.4) (width 0.2) (layer "B.Cu") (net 20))
 (segment (start 54.88 77.5) (end 45.66 68.28) (width 0.2) (layer "B.Cu") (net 20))
 (segment (start 45.66 58.688628) (end 46.94863 57.4) (width 0.2) (layer "B.Cu") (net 20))
 (segment (start 45.66 68.28) (end 45.66 58.688628) (width 0.2) (layer "B.Cu") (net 20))
 (segment (start 50.28 57.4) (end 55.18 52.5) (width 0.2) (layer "B.Cu") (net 20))
 (segment (start 60.54 57.3) (end 57.72 60.12) (width 0.2) (layer "F.Cu") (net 7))
 (segment (start 87.9 77.5) (end 83.62 73.22) (width 0.2) (layer "F.Cu") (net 7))
 (segment (start 82.431371 57.3) (end 60.54 57.3) (width 0.2) (layer "F.Cu") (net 7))
 (segment (start 83.619999 58.488629) (end 82.431371 57.3) (width 0.2) (layer "F.Cu") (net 7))
 (segment (start 83.62 73.22) (end 83.619999 58.488629) (width 0.2) (layer "F.Cu") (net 7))
 (segment (start 69.15 75.93) (end 69.15 58.85) (width 0.2) (layer "B.Cu") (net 15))
 (segment (start 69.15 58.85) (end 75.5 52.5) (width 0.2) (layer "B.Cu") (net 15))
 (segment (start 67.58 77.5) (end 69.15 75.93) (width 0.2) (layer "B.Cu") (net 15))
 (segment (start 81.5 72) (end 81.5 61.04) (width 0.2) (layer "F.Cu") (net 12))
 (segment (start 76 77.5) (end 81.5 72) (width 0.2) (layer "F.Cu") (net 12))
 (segment (start 81.5 61.04) (end 80.58 60.12) (width 0.2) (layer "F.Cu") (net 12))
 (segment (start 75.2 77.5) (end 76 77.5) (width 0.2) (layer "F.Cu") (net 12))
 (segment (start 71.65 58.89) (end 78.04 52.5) (width 0.2) (layer "B.Cu") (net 14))
 (segment (start 71.65 75.97) (end 71.65 58.89) (width 0.2) (layer "B.Cu") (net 14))
 (segment (start 70.12 77.5) (end 71.65 75.97) (width 0.2) (layer "B.Cu") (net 14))
 (segment (start 81.768628 58.9) (end 79.26 58.9) (width 0.2) (layer "F.Cu") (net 11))
 (segment (start 79.26 58.9) (end 78.04 60.12) (width 0.2) (layer "F.Cu") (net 11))
 (segment (start 82 59.131372) (end 81.768628 58.9) (width 0.2) (layer "F.Cu") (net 11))
 (segment (start 78.5 77.5) (end 82 74) (width 0.2) (layer "F.Cu") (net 11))
 (segment (start 82 74) (end 82 59.131372) (width 0.2) (layer "F.Cu") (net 11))
 (segment (start 77.74 77.5) (end 78.5 77.5) (width 0.2) (layer "F.Cu") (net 11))
 (segment (start 77.12 58.5) (end 75.5 60.12) (width 0.2) (layer "F.Cu") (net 10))
 (segment (start 82.42 75.36) (end 82.42 58.985687) (width 0.2) (layer "F.Cu") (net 10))
 (segment (start 80.28 77.5) (end 82.42 75.36) (width 0.2) (layer "F.Cu") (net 10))
 (segment (start 81.934313 58.5) (end 77.12 58.5) (width 0.2) (layer "F.Cu") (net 10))
 (segment (start 82.42 58.985687) (end 81.934313 58.5) (width 0.2) (layer "F.Cu") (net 10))
 (segment (start 49.8 77.5) (end 44.860001 72.560001) (width 0.2) (layer "B.Cu") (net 22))
 (segment (start 44.860001 57.739999) (end 50.1 52.5) (width 0.2) (layer "B.Cu") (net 22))
 (segment (start 44.860001 72.560001) (end 44.860001 57.739999) (width 0.2) (layer "B.Cu") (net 22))
 (segment (start 74.98 58.1) (end 72.96 60.12) (width 0.2) (layer "F.Cu") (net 9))
 (segment (start 82.82 58.820001) (end 82.099998 58.1) (width 0.2) (layer "F.Cu") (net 9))
 (segment (start 82.099998 58.1) (end 74.98 58.1) (width 0.2) (layer "F.Cu") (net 9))
 (segment (start 82.82 77.5) (end 82.82 58.820001) (width 0.2) (layer "F.Cu") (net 9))
 (segment (start 48.14 57) (end 52.64 52.5) (width 0.2) (layer "B.Cu") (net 21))
 (segment (start 45.260001 58.522942) (end 46.782945 57) (width 0.2) (layer "B.Cu") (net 21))
 (segment (start 45.260001 70.420001) (end 45.260001 58.522942) (width 0.2) (layer "B.Cu") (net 21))
 (segment (start 46.782945 57) (end 48.14 57) (width 0.2) (layer "B.Cu") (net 21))
 (segment (start 52.34 77.5) (end 45.260001 70.420001) (width 0.2) (layer "B.Cu") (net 21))
 (segment (start 74.06 76.1) (end 74.06 59.02) (width 0.2) (layer "B.Cu") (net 13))
 (segment (start 72.66 77.5) (end 74.06 76.1) (width 0.2) (layer "B.Cu") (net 13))
 (segment (start 74.06 59.02) (end 80.58 52.5) (width 0.2) (layer "B.Cu") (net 13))
 (segment (start 66.78 75.76) (end 66.78 58.68) (width 0.2) (layer "B.Cu") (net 16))
 (segment (start 66.78 58.68) (end 72.96 52.5) (width 0.2) (layer "B.Cu") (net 16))
 (segment (start 65.04 77.5) (end 66.78 75.76) (width 0.2) (layer "B.Cu") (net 16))
 (segment (start 85.36 77.5) (end 83.22 75.36) (width 0.2) (layer "F.Cu") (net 8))
 (segment (start 82.265683 57.7) (end 62.68 57.7) (width 0.2) (layer "F.Cu") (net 8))
 (segment (start 83.22 58.654315) (end 82.265683 57.7) (width 0.2) (layer "F.Cu") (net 8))
 (segment (start 62.68 57.7) (end 60.26 60.12) (width 0.2) (layer "F.Cu") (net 8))
 (segment (start 83.22 75.36) (end 83.22 58.654315) (width 0.2) (layer "F.Cu") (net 8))
 (segment (start 46.46 59.02) (end 47.28 58.2) (width 0.2) (layer "B.Cu") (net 18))
 (segment (start 47.28 58.2) (end 54.56 58.2) (width 0.2) (layer "B.Cu") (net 18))
 (segment (start 54.56 58.2) (end 60.26 52.5) (width 0.2) (layer "B.Cu") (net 18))
 (segment (start 59.96 77.5) (end 46.46 64) (width 0.2) (layer "B.Cu") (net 18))
 (segment (start 46.46 64) (end 46.46 59.02) (width 0.2) (layer "B.Cu") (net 18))
 (segment (start 72.02 62.02) (end 69.78 62.02) (width 0.2) (layer "F.Cu") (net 26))
 (segment (start 74 64) (end 72.02 62.02) (width 0.2) (layer "F.Cu") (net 26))
 (segment (start 69.78 62.02) (end 67.88 60.12) (width 0.2) (layer "F.Cu") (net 26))
 (segment (start 79 64) (end 76.22 61.22) (width 0.2) (layer "F.Cu") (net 27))
 (segment (start 71.52 61.22) (end 70.42 60.12) (width 0.2) (layer "F.Cu") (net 27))
 (segment (start 76.22 61.22) (end 71.52 61.22) (width 0.2) (layer "F.Cu") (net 27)))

